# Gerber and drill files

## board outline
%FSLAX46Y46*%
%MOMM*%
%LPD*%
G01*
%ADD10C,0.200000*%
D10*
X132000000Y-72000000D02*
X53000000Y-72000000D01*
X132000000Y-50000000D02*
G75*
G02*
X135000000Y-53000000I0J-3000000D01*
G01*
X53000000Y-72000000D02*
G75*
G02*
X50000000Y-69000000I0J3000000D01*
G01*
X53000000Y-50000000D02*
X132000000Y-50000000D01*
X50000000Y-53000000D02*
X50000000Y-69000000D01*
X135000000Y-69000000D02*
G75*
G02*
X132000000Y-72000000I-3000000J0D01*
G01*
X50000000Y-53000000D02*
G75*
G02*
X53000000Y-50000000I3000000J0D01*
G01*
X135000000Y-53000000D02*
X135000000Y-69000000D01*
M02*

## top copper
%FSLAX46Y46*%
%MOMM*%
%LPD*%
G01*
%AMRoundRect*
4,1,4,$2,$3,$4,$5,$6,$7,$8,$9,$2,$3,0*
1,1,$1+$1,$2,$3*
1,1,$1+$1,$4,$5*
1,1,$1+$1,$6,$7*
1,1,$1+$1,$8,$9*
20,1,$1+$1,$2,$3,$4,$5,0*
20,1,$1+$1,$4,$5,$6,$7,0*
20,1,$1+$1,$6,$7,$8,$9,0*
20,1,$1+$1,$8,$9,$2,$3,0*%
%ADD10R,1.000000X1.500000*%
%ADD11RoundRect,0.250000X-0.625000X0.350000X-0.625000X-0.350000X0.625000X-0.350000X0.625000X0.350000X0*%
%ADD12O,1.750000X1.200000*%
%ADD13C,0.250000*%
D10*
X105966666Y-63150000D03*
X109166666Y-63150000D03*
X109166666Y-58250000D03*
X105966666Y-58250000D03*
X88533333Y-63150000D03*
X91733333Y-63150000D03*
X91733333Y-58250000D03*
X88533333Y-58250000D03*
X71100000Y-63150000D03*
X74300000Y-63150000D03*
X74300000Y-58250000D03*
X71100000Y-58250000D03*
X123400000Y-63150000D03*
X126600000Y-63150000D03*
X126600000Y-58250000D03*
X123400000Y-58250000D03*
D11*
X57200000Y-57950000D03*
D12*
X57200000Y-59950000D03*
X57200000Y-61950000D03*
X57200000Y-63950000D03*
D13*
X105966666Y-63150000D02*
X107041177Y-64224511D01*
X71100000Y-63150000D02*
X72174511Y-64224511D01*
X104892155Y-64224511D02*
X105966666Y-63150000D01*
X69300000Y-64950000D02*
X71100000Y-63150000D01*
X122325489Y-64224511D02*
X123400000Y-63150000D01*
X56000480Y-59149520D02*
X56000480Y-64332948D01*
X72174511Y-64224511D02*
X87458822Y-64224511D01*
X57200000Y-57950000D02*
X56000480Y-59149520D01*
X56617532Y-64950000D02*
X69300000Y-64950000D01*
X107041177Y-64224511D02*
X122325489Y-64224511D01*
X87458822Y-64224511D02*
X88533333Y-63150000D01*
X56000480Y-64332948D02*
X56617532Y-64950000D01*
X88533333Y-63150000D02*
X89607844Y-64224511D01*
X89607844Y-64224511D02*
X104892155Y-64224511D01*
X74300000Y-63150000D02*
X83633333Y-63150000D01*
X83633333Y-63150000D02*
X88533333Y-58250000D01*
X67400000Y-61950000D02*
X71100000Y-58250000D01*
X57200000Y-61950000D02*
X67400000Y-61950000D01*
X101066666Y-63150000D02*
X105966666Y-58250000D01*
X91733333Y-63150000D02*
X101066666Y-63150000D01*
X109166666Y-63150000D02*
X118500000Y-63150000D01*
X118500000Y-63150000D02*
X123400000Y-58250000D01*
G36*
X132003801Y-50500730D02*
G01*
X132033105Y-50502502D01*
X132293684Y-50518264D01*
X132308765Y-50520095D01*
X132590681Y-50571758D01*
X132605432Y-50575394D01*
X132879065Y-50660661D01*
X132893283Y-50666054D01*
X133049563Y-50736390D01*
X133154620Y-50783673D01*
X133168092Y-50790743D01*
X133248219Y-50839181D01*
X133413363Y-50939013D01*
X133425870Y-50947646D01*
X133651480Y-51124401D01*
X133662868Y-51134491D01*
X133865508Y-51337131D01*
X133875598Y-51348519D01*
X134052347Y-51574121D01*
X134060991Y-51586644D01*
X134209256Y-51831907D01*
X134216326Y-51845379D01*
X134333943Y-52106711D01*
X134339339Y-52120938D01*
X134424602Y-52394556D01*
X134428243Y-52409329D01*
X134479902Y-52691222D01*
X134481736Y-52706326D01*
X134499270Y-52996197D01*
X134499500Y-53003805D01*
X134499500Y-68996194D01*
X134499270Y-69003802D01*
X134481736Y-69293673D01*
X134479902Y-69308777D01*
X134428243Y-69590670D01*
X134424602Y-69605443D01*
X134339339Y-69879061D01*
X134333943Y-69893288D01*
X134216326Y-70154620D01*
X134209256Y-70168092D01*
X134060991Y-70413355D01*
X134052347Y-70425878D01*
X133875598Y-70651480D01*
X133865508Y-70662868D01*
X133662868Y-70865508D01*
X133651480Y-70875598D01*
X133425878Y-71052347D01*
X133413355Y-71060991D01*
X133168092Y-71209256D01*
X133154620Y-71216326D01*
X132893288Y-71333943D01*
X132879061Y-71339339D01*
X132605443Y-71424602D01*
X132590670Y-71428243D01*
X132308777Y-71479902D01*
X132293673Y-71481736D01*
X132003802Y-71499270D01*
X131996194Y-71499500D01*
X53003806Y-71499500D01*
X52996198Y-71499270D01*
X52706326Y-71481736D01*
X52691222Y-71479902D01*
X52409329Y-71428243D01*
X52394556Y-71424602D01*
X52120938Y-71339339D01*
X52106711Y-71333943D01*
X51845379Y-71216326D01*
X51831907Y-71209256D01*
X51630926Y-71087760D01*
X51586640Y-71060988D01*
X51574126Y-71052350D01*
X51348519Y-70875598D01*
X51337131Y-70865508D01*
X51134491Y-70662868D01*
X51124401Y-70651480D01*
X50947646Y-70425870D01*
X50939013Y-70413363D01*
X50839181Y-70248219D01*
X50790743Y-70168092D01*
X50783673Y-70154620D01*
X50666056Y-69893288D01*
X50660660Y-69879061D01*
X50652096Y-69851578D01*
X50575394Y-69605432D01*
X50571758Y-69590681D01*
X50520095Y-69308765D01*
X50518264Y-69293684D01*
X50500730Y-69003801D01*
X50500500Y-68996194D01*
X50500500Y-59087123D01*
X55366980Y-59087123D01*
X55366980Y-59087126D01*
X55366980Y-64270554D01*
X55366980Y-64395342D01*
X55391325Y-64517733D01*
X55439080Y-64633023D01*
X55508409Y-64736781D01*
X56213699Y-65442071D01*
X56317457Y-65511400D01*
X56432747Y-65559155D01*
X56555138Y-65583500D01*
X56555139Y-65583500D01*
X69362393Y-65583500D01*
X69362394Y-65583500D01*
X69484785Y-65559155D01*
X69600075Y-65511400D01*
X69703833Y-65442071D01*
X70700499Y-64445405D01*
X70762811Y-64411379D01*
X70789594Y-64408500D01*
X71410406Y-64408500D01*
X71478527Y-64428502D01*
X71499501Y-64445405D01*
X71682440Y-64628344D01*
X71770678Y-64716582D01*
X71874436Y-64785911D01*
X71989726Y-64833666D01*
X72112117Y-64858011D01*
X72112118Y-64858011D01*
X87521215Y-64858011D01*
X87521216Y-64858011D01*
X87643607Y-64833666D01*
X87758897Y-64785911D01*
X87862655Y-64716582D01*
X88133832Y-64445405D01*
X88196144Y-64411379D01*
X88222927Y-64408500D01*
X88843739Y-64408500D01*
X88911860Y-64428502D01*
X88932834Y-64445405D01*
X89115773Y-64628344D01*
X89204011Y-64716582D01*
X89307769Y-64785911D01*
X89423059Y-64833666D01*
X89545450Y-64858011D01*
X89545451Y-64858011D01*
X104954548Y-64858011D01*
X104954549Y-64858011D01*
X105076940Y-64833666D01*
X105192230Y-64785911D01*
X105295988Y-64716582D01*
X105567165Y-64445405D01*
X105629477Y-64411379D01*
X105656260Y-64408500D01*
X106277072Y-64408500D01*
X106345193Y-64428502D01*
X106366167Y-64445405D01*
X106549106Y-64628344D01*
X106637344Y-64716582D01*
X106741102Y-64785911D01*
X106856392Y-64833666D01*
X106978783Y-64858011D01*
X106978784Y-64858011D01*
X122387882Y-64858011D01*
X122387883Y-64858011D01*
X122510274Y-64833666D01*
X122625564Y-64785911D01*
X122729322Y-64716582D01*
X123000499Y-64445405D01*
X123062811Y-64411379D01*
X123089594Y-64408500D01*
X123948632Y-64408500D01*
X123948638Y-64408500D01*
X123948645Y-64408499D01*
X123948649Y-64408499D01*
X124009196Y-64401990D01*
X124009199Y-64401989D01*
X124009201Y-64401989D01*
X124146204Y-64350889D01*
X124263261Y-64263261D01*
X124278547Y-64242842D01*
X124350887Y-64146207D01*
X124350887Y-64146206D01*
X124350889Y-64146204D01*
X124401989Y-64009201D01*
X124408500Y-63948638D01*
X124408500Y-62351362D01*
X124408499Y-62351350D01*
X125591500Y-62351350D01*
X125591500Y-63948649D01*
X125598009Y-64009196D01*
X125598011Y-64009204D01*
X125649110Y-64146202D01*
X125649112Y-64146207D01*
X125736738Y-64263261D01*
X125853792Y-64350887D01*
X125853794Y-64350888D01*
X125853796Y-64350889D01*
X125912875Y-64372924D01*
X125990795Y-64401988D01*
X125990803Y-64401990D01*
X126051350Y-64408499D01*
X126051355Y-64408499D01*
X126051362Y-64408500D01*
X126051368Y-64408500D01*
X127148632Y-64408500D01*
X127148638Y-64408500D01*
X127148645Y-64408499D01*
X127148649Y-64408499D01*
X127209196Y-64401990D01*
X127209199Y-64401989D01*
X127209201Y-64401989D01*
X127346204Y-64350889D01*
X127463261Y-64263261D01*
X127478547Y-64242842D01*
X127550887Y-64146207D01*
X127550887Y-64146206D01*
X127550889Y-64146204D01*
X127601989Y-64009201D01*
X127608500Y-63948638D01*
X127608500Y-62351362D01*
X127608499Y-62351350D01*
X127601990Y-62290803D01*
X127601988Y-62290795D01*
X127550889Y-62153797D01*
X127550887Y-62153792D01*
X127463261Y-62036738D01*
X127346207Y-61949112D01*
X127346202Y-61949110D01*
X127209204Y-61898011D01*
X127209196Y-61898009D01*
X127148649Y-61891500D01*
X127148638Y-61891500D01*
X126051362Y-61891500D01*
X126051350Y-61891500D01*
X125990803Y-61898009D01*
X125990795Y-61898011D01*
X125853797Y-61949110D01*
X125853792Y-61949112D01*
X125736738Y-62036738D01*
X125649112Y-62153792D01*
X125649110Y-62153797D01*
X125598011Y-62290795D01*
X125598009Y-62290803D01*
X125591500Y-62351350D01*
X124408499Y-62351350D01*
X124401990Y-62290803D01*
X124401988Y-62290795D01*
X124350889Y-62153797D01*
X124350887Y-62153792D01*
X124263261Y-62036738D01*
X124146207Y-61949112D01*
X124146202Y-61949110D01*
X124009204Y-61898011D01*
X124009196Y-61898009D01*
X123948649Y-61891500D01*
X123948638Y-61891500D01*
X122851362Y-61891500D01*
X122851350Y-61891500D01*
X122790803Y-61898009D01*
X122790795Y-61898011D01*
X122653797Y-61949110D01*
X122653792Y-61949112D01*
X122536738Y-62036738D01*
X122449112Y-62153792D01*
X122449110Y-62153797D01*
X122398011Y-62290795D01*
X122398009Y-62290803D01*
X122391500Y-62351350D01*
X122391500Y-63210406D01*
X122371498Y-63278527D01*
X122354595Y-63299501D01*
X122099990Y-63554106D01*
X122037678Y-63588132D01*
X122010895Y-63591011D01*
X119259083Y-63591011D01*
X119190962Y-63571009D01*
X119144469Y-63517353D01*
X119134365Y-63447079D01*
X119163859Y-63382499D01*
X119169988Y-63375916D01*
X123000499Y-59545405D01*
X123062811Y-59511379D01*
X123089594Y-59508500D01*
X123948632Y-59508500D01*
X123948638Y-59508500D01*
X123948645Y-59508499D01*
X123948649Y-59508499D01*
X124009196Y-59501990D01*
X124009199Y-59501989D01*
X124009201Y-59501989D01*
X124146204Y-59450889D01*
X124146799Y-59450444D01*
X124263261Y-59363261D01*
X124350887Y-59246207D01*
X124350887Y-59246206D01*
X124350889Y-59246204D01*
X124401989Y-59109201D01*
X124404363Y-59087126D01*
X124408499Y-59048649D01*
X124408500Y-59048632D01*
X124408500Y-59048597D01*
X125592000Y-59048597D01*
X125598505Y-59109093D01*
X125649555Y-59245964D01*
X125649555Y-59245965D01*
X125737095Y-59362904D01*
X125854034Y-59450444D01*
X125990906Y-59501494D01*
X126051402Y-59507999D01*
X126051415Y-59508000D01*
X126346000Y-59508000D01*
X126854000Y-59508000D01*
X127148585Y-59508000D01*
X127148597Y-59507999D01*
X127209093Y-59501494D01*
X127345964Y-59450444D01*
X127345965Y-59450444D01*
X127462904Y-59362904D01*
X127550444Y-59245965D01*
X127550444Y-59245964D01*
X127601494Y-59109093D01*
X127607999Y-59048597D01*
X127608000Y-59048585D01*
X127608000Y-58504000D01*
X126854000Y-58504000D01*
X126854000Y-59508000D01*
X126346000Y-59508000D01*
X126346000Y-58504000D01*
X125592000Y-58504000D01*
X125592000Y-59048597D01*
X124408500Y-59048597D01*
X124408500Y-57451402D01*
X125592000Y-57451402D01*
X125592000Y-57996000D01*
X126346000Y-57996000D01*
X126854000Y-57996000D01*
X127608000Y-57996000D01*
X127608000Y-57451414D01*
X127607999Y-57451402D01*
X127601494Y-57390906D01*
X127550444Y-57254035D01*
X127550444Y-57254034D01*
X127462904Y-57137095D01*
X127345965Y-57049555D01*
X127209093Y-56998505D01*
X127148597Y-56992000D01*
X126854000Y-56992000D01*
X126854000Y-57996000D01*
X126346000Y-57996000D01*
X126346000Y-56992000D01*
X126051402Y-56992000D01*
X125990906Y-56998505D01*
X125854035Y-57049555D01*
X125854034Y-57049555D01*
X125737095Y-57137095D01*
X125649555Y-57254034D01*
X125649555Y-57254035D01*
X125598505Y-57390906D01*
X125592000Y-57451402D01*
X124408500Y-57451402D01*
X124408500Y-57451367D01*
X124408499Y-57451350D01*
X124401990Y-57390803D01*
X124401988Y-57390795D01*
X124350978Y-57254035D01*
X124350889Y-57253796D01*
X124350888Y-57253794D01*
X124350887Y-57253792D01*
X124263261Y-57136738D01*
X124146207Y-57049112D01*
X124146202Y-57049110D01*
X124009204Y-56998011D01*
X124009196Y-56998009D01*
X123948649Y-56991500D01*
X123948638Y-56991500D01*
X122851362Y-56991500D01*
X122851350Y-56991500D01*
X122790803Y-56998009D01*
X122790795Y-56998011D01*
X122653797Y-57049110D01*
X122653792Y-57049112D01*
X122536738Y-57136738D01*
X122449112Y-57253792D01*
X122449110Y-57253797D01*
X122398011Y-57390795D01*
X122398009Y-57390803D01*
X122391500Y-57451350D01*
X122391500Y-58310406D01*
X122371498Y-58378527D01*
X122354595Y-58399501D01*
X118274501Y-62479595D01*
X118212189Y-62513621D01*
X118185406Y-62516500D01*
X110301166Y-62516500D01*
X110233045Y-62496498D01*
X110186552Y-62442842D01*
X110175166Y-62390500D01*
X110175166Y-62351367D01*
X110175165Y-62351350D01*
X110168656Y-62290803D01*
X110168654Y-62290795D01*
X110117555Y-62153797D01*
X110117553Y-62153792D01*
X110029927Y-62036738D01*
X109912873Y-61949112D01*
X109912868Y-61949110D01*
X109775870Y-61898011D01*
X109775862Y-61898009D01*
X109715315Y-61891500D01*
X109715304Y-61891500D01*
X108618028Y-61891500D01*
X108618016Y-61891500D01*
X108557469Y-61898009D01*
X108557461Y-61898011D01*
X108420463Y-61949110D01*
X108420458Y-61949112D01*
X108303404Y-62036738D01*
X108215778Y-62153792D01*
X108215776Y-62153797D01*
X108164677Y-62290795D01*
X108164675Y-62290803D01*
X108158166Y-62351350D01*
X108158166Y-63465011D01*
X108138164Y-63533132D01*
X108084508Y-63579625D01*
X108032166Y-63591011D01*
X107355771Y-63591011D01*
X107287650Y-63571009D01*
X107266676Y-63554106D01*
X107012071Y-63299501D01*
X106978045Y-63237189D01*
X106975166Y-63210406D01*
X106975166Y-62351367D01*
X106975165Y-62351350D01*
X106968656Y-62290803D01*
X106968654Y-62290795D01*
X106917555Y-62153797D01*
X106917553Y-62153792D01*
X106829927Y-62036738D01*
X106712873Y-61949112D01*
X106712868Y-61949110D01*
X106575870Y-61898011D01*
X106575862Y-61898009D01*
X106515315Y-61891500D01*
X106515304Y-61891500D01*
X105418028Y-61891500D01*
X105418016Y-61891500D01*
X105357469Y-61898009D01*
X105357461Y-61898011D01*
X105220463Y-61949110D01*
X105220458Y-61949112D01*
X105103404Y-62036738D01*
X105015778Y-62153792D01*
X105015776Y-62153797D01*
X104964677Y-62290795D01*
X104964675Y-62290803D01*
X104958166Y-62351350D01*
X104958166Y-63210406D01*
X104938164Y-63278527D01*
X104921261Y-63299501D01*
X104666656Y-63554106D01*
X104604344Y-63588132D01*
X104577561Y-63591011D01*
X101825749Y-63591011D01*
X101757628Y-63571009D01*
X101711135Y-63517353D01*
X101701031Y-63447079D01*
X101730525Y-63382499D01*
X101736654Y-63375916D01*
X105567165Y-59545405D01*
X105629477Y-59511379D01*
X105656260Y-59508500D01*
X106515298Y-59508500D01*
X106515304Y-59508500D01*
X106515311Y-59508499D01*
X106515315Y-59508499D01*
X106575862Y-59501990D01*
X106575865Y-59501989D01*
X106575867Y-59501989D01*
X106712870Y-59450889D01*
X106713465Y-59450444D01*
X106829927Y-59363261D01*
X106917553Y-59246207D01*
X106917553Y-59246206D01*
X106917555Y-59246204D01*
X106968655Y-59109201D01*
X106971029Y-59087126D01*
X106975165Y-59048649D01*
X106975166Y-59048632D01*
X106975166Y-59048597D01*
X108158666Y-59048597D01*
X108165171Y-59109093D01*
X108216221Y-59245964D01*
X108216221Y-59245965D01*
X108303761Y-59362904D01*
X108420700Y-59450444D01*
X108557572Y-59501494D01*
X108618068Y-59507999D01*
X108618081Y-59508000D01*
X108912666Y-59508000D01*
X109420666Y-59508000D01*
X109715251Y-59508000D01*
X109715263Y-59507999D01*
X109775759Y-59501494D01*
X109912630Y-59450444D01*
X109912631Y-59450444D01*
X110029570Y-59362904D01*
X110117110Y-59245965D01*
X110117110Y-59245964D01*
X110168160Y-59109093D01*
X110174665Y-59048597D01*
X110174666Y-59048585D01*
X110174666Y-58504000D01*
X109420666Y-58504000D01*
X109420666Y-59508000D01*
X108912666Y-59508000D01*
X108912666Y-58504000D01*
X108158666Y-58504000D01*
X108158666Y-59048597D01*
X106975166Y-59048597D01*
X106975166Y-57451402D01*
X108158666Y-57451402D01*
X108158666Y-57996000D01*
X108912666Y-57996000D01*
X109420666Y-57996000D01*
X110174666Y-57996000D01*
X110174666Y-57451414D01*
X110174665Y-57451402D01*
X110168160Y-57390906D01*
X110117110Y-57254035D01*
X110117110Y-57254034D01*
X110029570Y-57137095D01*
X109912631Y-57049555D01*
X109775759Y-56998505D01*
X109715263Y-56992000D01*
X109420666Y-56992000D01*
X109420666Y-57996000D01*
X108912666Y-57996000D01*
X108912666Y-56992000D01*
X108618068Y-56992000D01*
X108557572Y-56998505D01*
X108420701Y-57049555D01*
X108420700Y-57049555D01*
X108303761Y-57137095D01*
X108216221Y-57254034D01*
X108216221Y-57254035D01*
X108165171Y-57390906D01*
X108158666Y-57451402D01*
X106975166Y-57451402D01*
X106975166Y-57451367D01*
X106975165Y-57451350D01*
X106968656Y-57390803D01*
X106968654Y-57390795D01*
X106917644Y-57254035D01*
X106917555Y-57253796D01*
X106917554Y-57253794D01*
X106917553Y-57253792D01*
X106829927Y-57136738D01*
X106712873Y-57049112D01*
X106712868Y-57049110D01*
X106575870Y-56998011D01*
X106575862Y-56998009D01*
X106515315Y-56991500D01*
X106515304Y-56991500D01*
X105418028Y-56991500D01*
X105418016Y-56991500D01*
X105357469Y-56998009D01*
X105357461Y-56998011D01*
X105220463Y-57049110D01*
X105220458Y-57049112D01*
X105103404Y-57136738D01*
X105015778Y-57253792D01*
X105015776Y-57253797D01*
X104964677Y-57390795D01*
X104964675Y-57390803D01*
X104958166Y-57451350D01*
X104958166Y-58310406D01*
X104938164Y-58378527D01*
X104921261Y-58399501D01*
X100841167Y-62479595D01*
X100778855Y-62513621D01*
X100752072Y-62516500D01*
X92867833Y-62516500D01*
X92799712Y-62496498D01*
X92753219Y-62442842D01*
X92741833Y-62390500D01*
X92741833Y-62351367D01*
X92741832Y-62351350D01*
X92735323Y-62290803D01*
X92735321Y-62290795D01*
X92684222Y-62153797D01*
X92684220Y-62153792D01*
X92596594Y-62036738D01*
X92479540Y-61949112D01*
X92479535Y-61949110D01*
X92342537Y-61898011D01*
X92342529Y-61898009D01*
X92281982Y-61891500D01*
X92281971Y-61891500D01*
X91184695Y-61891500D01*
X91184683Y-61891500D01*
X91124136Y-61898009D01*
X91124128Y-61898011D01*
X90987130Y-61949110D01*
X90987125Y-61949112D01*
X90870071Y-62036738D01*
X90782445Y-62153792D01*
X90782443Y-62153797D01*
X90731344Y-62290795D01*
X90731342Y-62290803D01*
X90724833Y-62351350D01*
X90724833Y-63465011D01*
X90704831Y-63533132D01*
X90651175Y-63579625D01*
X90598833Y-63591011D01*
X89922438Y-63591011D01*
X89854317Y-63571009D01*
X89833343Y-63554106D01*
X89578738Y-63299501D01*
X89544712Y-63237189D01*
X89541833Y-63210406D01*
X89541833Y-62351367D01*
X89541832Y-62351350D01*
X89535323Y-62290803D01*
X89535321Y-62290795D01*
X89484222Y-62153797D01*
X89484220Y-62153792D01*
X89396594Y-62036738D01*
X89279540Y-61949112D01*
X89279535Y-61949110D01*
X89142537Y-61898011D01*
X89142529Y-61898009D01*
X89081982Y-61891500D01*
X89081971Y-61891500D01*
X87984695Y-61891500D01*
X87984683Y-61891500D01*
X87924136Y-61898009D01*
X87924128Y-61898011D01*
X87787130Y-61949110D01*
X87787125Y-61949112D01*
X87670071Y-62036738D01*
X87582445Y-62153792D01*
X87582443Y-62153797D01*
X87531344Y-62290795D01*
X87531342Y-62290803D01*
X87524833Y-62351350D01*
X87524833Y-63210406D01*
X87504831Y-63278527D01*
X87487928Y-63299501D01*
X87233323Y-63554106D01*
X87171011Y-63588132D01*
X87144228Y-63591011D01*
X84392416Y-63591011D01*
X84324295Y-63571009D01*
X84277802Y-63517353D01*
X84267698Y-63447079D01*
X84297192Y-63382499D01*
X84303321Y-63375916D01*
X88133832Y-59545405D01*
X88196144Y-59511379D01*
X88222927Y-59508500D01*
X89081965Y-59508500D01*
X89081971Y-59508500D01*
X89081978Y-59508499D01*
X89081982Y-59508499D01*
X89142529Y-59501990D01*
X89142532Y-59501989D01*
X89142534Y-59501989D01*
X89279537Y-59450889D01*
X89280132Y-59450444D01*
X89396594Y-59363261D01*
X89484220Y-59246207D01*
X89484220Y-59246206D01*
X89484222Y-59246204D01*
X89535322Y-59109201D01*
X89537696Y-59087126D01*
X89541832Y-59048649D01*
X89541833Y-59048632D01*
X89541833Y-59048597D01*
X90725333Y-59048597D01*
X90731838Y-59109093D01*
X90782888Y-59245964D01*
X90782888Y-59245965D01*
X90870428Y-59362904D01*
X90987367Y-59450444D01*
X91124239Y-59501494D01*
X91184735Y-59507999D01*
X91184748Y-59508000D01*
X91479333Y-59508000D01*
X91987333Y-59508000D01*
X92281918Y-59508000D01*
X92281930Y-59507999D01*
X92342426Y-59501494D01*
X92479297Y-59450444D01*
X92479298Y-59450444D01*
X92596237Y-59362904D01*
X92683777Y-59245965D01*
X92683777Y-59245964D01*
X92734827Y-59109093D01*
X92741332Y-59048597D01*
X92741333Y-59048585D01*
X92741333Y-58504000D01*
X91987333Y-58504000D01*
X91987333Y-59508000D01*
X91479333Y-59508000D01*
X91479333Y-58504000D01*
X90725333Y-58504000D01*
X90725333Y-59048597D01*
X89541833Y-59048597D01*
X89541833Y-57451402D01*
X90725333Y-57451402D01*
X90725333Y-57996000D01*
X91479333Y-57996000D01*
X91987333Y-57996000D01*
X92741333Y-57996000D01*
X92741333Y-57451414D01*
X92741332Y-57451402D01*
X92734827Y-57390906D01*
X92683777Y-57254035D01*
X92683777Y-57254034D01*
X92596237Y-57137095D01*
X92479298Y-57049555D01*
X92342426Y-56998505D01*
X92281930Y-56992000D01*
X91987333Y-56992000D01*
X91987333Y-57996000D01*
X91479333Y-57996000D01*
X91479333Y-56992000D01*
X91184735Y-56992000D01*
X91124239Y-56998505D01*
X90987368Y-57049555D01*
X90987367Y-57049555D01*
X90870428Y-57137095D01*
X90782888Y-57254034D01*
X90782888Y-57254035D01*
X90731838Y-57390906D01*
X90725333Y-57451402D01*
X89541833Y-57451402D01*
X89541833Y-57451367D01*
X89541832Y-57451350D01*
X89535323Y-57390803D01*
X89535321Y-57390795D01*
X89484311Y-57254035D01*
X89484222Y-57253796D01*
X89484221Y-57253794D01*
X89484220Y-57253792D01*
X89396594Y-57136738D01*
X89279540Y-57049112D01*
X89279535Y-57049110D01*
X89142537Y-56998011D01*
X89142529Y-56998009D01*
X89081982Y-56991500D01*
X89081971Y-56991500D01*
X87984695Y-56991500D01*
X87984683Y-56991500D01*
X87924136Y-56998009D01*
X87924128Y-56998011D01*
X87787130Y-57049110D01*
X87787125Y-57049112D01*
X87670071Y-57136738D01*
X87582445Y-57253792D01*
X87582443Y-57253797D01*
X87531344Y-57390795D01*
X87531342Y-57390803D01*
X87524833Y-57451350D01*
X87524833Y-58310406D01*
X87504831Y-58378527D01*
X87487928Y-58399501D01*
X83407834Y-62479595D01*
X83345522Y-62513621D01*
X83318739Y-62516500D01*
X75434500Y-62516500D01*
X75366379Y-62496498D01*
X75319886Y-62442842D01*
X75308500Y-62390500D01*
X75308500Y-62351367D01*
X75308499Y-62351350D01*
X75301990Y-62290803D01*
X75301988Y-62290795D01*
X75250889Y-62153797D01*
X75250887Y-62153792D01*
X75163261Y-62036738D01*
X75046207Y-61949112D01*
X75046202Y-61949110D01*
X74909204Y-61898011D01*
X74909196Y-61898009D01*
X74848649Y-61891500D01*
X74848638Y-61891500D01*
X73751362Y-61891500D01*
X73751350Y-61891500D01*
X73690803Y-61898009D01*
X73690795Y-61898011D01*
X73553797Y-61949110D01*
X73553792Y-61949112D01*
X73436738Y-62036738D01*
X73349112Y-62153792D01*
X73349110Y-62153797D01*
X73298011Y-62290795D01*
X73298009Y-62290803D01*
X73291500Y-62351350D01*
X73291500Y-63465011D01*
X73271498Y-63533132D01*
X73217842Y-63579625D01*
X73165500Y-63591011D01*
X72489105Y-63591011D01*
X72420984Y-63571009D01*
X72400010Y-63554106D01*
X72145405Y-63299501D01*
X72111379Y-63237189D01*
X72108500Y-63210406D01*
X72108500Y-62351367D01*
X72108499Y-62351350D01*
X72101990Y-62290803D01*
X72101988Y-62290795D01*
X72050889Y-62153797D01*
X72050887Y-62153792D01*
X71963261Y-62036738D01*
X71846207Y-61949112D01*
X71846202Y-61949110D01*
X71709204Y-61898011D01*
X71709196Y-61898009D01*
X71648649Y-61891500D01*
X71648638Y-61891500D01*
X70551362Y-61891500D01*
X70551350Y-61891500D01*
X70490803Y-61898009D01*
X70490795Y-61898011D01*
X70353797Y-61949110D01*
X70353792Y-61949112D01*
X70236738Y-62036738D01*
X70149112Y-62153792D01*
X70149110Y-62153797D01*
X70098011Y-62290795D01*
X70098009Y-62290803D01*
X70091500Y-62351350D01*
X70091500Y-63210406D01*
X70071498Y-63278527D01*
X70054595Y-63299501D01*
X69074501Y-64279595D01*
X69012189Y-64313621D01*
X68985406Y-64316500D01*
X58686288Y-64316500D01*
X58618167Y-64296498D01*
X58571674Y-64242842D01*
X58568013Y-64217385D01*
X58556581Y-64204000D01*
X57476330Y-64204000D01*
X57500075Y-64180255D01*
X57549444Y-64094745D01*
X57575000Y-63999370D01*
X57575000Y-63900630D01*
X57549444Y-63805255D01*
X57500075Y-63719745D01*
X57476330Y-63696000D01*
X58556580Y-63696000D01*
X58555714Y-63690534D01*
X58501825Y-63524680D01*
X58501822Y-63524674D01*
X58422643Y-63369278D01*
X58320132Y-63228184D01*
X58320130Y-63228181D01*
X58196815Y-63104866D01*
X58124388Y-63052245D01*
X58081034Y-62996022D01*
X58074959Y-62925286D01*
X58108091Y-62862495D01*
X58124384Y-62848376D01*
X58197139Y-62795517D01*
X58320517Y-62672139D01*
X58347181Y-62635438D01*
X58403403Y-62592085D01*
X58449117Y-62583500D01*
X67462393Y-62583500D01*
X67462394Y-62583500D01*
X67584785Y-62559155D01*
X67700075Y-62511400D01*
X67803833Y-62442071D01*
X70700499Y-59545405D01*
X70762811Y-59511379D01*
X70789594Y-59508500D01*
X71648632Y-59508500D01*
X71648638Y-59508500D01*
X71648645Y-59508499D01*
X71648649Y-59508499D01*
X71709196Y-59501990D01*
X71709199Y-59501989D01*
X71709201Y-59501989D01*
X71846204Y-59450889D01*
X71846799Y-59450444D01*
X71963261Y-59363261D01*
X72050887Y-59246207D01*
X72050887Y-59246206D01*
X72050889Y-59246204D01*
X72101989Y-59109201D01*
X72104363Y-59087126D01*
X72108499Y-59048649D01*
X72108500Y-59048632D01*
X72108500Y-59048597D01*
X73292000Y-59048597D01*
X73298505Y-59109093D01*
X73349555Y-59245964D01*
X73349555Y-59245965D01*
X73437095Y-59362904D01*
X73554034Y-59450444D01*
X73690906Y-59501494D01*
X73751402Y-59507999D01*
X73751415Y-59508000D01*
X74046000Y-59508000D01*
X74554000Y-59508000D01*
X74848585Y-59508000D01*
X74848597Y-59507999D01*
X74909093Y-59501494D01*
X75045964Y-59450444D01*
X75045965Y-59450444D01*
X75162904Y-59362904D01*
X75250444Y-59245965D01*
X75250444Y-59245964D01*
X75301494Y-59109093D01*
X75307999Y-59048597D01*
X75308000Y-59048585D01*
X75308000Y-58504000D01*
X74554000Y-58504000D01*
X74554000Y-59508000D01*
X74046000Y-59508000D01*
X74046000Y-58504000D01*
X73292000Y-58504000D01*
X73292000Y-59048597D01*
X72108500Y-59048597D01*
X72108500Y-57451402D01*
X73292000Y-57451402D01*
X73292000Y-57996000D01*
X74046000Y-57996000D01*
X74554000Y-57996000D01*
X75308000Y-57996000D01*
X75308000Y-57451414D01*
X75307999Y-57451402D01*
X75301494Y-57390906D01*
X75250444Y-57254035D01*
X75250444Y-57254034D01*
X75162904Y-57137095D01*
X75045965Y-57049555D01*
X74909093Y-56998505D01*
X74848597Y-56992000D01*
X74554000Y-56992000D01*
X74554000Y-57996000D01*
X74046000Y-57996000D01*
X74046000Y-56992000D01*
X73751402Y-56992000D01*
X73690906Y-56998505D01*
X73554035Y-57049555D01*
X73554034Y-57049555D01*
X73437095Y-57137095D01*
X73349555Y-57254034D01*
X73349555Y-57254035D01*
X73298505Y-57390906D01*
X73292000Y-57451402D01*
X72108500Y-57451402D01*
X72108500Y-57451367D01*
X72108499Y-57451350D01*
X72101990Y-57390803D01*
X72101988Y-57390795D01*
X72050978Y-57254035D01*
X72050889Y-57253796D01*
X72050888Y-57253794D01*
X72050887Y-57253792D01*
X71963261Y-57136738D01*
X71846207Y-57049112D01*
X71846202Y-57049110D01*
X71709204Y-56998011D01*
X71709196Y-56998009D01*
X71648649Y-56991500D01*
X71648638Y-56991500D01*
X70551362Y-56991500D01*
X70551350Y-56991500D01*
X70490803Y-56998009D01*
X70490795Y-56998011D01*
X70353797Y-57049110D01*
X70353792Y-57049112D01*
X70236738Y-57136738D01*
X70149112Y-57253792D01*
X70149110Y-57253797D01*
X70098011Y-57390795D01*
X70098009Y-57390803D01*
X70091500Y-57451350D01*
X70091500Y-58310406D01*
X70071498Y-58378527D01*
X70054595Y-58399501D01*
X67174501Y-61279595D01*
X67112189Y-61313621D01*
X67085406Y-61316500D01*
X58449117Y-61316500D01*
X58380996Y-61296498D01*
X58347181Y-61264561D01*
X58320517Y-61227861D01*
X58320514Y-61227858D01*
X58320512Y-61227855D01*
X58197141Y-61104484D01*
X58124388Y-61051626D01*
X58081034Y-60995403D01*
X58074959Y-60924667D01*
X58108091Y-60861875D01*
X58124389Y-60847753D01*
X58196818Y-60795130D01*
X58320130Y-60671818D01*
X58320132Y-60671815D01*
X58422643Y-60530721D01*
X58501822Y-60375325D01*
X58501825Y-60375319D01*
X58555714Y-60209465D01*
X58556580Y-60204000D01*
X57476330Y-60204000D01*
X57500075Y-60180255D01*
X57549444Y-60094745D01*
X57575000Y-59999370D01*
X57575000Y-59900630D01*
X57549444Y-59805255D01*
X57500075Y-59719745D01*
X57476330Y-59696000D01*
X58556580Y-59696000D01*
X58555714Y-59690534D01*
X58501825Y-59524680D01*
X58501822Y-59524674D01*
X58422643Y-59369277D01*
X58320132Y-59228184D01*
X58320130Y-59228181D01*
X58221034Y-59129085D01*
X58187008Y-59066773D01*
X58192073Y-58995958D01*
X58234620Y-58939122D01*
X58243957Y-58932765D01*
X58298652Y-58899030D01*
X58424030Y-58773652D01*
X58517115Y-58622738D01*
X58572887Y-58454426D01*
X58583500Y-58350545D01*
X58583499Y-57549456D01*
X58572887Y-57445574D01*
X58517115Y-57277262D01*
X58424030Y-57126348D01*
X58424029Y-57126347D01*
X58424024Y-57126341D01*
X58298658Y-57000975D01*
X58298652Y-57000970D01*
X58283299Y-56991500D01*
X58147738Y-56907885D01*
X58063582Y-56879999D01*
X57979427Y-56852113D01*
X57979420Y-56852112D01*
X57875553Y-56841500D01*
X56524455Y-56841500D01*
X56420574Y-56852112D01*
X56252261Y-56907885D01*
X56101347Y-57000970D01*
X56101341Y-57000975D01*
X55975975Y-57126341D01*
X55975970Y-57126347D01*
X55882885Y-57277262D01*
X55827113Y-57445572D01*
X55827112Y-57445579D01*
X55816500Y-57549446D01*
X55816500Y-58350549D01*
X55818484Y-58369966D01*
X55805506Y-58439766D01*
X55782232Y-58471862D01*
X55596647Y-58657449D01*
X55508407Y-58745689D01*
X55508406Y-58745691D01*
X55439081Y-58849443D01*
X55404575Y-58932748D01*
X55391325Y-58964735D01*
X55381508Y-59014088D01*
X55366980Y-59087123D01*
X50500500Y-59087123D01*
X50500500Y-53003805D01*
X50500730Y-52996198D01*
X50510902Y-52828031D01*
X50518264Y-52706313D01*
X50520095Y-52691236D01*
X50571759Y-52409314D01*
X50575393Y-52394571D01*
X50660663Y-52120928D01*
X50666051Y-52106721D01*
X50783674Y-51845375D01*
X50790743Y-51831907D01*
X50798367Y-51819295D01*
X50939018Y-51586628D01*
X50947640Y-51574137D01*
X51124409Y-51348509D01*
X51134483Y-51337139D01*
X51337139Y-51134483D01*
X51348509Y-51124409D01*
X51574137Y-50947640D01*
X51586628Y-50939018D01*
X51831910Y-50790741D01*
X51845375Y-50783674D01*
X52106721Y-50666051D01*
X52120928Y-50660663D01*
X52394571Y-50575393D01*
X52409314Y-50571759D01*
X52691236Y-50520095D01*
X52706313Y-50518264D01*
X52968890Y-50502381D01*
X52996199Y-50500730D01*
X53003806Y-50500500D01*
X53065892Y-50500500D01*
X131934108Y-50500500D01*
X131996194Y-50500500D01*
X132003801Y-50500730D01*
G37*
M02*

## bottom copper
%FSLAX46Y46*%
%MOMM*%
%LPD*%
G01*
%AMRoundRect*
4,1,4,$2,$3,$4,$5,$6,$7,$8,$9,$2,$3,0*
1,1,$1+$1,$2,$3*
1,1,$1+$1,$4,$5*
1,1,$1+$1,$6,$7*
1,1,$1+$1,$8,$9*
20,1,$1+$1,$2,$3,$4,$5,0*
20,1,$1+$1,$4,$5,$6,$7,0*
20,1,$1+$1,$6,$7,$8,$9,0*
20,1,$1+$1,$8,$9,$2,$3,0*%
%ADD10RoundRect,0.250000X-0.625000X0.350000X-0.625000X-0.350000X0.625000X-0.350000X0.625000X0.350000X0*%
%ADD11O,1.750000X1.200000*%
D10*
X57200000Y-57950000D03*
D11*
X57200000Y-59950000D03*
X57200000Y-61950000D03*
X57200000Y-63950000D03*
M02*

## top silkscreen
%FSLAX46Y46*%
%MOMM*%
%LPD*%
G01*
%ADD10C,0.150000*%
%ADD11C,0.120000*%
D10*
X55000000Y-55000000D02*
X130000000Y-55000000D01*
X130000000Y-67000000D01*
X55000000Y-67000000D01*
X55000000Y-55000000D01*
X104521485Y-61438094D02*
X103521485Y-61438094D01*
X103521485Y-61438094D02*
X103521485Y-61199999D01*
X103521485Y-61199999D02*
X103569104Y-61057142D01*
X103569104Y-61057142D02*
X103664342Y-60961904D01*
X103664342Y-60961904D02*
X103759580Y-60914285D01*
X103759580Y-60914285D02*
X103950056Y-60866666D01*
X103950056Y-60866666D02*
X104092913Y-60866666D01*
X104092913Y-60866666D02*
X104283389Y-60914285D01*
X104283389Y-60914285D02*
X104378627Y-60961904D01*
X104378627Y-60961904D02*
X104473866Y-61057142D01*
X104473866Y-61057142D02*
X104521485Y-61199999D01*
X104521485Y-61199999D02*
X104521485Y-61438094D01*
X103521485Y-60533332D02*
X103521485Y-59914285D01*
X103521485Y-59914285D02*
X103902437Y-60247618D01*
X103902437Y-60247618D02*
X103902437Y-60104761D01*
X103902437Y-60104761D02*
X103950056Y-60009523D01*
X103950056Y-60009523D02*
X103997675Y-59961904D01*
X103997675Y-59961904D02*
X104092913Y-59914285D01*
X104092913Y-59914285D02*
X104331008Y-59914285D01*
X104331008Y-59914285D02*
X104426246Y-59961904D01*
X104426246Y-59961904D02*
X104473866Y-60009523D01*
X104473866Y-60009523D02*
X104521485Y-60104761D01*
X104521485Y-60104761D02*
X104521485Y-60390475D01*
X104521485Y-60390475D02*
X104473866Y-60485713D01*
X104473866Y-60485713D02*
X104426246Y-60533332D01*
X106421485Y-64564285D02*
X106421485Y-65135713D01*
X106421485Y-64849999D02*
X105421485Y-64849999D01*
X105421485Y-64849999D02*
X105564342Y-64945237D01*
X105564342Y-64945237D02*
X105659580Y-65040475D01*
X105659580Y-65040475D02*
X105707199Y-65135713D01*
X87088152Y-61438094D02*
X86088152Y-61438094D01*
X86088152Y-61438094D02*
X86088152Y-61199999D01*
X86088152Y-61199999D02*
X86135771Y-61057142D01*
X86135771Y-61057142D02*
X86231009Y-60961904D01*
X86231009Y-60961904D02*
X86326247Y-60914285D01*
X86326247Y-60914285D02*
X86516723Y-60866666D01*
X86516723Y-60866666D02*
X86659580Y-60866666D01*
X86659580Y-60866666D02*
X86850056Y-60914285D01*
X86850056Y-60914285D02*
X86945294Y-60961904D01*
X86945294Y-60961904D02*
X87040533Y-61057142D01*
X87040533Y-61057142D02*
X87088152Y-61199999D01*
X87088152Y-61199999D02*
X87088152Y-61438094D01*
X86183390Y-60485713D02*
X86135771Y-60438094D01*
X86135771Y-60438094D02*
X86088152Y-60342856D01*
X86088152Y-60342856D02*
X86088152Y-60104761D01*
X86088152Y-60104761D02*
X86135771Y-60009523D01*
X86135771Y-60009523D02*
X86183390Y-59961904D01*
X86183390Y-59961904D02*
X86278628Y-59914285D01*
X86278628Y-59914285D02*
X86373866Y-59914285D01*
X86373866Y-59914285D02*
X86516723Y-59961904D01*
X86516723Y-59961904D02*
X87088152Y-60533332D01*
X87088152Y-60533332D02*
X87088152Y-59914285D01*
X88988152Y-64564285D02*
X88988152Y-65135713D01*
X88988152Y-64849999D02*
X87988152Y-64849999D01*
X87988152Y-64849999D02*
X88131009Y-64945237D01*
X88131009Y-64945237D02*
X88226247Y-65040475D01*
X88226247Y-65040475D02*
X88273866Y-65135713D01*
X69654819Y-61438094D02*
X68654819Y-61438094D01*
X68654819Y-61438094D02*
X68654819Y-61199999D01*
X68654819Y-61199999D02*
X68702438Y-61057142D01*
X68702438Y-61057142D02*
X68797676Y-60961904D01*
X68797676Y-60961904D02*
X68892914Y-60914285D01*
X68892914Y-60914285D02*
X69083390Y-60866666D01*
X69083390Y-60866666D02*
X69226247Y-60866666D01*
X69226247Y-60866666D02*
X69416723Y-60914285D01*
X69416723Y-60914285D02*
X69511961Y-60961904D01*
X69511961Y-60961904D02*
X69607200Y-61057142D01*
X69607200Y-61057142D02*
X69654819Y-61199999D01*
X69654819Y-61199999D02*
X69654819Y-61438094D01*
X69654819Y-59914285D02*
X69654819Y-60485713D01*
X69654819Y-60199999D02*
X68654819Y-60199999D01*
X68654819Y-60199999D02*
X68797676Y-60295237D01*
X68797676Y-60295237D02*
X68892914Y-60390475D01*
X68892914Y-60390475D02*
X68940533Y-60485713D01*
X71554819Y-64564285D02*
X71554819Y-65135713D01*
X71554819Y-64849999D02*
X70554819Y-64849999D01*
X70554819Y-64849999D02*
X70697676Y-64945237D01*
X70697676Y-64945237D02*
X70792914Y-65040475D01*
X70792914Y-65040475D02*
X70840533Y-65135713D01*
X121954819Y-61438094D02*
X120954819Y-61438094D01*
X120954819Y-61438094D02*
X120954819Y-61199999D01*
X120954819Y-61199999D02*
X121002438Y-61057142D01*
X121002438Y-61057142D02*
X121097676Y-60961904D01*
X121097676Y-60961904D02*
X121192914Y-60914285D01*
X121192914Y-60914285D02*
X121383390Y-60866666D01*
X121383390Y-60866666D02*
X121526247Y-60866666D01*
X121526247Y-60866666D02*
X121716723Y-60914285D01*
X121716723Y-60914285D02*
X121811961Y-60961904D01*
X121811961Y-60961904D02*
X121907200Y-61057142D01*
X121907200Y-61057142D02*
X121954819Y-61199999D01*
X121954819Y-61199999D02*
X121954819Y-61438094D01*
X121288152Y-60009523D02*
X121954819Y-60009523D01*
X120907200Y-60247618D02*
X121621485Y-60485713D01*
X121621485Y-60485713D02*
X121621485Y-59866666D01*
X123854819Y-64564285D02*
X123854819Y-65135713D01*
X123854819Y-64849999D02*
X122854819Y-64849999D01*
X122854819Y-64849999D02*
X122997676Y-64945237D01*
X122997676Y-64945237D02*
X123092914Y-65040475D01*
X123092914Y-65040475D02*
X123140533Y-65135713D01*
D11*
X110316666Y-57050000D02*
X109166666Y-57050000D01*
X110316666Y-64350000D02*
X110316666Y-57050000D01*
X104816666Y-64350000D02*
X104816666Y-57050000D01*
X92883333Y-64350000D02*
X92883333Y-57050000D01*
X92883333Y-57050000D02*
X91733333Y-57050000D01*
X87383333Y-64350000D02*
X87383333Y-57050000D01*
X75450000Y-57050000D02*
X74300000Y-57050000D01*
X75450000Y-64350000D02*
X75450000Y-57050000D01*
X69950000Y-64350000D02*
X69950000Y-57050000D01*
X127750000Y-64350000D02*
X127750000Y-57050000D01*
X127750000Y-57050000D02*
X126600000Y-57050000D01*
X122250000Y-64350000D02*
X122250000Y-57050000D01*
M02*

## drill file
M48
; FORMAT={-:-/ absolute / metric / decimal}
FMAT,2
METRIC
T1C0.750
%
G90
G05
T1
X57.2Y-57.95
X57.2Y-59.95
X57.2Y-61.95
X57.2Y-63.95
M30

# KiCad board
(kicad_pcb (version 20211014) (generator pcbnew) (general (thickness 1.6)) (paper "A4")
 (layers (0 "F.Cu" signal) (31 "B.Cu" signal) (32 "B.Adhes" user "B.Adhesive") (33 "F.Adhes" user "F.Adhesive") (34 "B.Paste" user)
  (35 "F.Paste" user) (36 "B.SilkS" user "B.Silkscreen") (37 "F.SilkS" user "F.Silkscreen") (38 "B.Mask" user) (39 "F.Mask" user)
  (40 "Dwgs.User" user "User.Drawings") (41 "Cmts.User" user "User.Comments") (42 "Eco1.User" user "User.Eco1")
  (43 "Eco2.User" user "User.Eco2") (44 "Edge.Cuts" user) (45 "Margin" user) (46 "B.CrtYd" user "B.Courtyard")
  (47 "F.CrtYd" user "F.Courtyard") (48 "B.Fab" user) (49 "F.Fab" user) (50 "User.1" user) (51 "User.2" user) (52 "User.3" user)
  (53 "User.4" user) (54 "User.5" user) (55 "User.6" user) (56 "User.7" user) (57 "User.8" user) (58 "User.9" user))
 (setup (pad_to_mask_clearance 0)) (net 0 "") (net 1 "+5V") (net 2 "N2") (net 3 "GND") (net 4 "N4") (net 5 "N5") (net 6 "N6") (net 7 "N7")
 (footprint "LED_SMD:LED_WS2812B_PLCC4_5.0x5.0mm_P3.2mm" (layer "F.Cu") (at 107.566666 60.7 90)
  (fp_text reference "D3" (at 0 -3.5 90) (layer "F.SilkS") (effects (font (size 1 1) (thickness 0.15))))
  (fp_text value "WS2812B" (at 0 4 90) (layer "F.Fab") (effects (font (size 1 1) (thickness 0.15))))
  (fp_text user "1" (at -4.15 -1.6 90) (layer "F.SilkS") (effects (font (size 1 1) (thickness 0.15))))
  (fp_line (start 3.65 2.75) (end 3.65 1.6) (layer "F.SilkS") (width 0.12))
  (fp_line (start -3.65 2.75) (end 3.65 2.75) (layer "F.SilkS") (width 0.12))
  (fp_line (start -3.65 -2.75) (end 3.65 -2.75) (layer "F.SilkS") (width 0.12))
  (pad "1" smd rect (at -2.45 -1.6 90) (size 1.5 1) (layers "F.Cu" "F.Paste" "F.Mask") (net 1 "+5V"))
  (pad "2" smd rect (at -2.45 1.6 90) (size 1.5 1) (layers "F.Cu" "F.Paste" "F.Mask") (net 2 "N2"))
  (pad "3" smd rect (at 2.45 1.6 90) (size 1.5 1) (layers "F.Cu" "F.Paste" "F.Mask") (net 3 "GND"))
  (pad "4" smd rect (at 2.45 -1.6 90) (size 1.5 1) (layers "F.Cu" "F.Paste" "F.Mask") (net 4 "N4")))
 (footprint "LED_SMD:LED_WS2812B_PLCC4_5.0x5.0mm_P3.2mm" (layer "F.Cu") (at 90.133333 60.7 90)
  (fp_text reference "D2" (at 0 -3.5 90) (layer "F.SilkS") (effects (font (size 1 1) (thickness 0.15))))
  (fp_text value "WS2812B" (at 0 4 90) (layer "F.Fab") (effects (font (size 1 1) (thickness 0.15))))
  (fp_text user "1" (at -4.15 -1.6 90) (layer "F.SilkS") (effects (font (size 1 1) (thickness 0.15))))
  (fp_line (start -3.65 2.75) (end 3.65 2.75) (layer "F.SilkS") (width 0.12))
  (fp_line (start 3.65 2.75) (end 3.65 1.6) (layer "F.SilkS") (width 0.12))
  (fp_line (start -3.65 -2.75) (end 3.65 -2.75) (layer "F.SilkS") (width 0.12))
  (pad "1" smd rect (at -2.45 -1.6 90) (size 1.5 1) (layers "F.Cu" "F.Paste" "F.Mask") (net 1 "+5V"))
  (pad "2" smd rect (at -2.45 1.6 90) (size 1.5 1) (layers "F.Cu" "F.Paste" "F.Mask") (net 4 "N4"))
  (pad "3" smd rect (at 2.45 1.6 90) (size 1.5 1) (layers "F.Cu" "F.Paste" "F.Mask") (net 3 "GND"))
  (pad "4" smd rect (at 2.45 -1.6 90) (size 1.5 1) (layers "F.Cu" "F.Paste" "F.Mask") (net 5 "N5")))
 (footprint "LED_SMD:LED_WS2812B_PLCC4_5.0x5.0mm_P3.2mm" (layer "F.Cu") (at 72.7 60.7 90)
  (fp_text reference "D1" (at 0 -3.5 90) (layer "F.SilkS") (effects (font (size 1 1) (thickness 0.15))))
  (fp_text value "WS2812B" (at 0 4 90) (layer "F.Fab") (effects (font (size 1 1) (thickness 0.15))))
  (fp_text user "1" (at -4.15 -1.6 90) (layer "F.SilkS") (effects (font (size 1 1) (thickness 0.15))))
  (fp_line (start 3.65 2.75) (end 3.65 1.6) (layer "F.SilkS") (width 0.12))
  (fp_line (start -3.65 2.75) (end 3.65 2.75) (layer "F.SilkS") (width 0.12))
  (fp_line (start -3.65 -2.75) (end 3.65 -2.75) (layer "F.SilkS") (width 0.12))
  (pad "1" smd rect (at -2.45 -1.6 90) (size 1.5 1) (layers "F.Cu" "F.Paste" "F.Mask") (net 1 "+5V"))
  (pad "2" smd rect (at -2.45 1.6 90) (size 1.5 1) (layers "F.Cu" "F.Paste" "F.Mask") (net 5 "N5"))
  (pad "3" smd rect (at 2.45 1.6 90) (size 1.5 1) (layers "F.Cu" "F.Paste" "F.Mask") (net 3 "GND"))
  (pad "4" smd rect (at 2.45 -1.6 90) (size 1.5 1) (layers "F.Cu" "F.Paste" "F.Mask") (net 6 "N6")))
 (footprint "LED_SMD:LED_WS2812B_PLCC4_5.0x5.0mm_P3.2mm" (layer "F.Cu") (at 125 60.7 90)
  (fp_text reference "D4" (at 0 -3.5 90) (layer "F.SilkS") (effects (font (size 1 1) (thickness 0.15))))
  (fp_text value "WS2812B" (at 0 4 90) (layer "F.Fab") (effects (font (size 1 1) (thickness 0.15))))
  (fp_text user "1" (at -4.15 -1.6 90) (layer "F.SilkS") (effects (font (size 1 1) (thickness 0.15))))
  (fp_line (start -3.65 2.75) (end 3.65 2.75) (layer "F.SilkS") (width 0.12))
  (fp_line (start 3.65 2.75) (end 3.65 1.6) (layer "F.SilkS") (width 0.12))
  (fp_line (start -3.65 -2.75) (end 3.65 -2.75) (layer "F.SilkS") (width 0.12))
  (pad "1" smd rect (at -2.45 -1.6 90) (size 1.5 1) (layers "F.Cu" "F.Paste" "F.Mask") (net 1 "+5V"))
  (pad "2" smd rect (at -2.45 1.6 90) (size 1.5 1) (layers "F.Cu" "F.Paste" "F.Mask") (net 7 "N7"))
  (pad "3" smd rect (at 2.45 1.6 90) (size 1.5 1) (layers "F.Cu" "F.Paste" "F.Mask") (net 3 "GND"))
  (pad "4" smd rect (at 2.45 -1.6 90) (size 1.5 1) (layers "F.Cu" "F.Paste" "F.Mask") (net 2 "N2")))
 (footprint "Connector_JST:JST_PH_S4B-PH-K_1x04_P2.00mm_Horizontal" (layer "B.Cu") (at 57.2 57.95 -90)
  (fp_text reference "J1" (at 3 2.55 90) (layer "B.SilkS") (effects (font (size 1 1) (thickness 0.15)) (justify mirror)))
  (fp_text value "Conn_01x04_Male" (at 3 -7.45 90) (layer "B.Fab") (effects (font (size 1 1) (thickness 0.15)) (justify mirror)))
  (pad "1" thru_hole roundrect (at 0 0 270) (size 1.2 1.75) (drill 0.75) (layers *.Cu *.Mask) (roundrect_rratio 0.208333) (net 1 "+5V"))
  (pad "2" thru_hole oval (at 2 0 270) (size 1.2 1.75) (drill 0.75) (layers *.Cu *.Mask) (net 3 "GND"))
  (pad "3" thru_hole oval (at 4 0 270) (size 1.2 1.75) (drill 0.75) (layers *.Cu *.Mask) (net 6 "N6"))
  (pad "4" thru_hole oval (at 6 0 270) (size 1.2 1.75) (drill 0.75) (layers *.Cu *.Mask) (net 3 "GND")))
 (gr_rect (start 55 55) (end 130 67) (layer "F.SilkS") (width 0.15) (fill none))
 (gr_line (start 132 72) (end 53 72) (layer "Edge.Cuts") (width 0.2))
 (gr_arc (start 132 50) (mid 134.12132 50.87868) (end 135 53) (layer "Edge.Cuts") (width 0.2))
 (gr_arc (start 53 72) (mid 50.87868 71.12132) (end 50 69) (layer "Edge.Cuts") (width 0.2))
 (gr_line (start 53 50) (end 132 50) (layer "Edge.Cuts") (width 0.2))
 (gr_line (start 50 53) (end 50 69) (layer "Edge.Cuts") (width 0.2))
 (gr_arc (start 135 69) (mid 134.12132 71.12132) (end 132 72) (layer "Edge.Cuts") (width 0.2))
 (gr_arc (start 50 53) (mid 50.87868 50.87868) (end 53 50) (layer "Edge.Cuts") (width 0.2))
 (gr_line (start 135 53) (end 135 69) (layer "Edge.Cuts") (width 0.2))
 (segment (start 105.966666 63.15) (end 107.041177 64.224511) (width 0.25) (layer "F.Cu") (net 1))
 (segment (start 71.1 63.15) (end 72.174511 64.224511) (width 0.25) (layer "F.Cu") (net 1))
 (segment (start 104.892155 64.224511) (end 105.966666 63.15) (width 0.25) (layer "F.Cu") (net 1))
 (segment (start 69.3 64.95) (end 71.1 63.15) (width 0.25) (layer "F.Cu") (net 1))
 (segment (start 122.325489 64.224511) (end 123.4 63.15) (width 0.25) (layer "F.Cu") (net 1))
 (segment (start 56.00048 59.14952) (end 56.00048 64.332948) (width 0.25) (layer "F.Cu") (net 1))
 (segment (start 72.174511 64.224511) (end 87.458822 64.224511) (width 0.25) (layer "F.Cu") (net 1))
 (segment (start 57.2 57.95) (end 56.00048 59.14952) (width 0.25) (layer "F.Cu") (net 1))
 (segment (start 56.617532 64.95) (end 69.3 64.95) (width 0.25) (layer "F.Cu") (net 1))
 (segment (start 107.041177 64.224511) (end 122.325489 64.224511) (width 0.25) (layer "F.Cu") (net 1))
 (segment (start 87.458822 64.224511) (end 88.533333 63.15) (width 0.25) (layer "F.Cu") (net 1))
 (segment (start 56.00048 64.332948) (end 56.617532 64.95) (width 0.25) (layer "F.Cu") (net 1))
 (segment (start 88.533333 63.15) (end 89.607844 64.224511) (width 0.25) (layer "F.Cu") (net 1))
 (segment (start 89.607844 64.224511) (end 104.892155 64.224511) (width 0.25) (layer "F.Cu") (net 1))
 (segment (start 74.3 63.15) (end 83.633333 63.15) (width 0.25) (layer "F.Cu") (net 5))
 (segment (start 83.633333 63.15) (end 88.533333 58.25) (width 0.25) (layer "F.Cu") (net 5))
 (segment (start 67.4 61.95) (end 71.1 58.25) (width 0.25) (layer "F.Cu") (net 6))
 (segment (start 57.2 61.95) (end 67.4 61.95) (width 0.25) (layer "F.Cu") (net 6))
 (segment (start 101.066666 63.15) (end 105.966666 58.25) (width 0.25) (layer "F.Cu") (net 4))
 (segment (start 91.733333 63.15) (end 101.066666 63.15) (width 0.25) (layer "F.Cu") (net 4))
 (segment (start 109.166666 63.15) (end 118.5 63.15) (width 0.25) (layer "F.Cu") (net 2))
 (segment (start 118.5 63.15) (end 123.4 58.25) (width 0.25) (layer "F.Cu") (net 2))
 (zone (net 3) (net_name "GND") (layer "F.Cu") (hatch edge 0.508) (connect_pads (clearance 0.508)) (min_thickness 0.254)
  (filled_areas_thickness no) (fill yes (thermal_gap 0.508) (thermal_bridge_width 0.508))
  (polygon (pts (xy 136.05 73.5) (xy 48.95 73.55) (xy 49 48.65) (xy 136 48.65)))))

